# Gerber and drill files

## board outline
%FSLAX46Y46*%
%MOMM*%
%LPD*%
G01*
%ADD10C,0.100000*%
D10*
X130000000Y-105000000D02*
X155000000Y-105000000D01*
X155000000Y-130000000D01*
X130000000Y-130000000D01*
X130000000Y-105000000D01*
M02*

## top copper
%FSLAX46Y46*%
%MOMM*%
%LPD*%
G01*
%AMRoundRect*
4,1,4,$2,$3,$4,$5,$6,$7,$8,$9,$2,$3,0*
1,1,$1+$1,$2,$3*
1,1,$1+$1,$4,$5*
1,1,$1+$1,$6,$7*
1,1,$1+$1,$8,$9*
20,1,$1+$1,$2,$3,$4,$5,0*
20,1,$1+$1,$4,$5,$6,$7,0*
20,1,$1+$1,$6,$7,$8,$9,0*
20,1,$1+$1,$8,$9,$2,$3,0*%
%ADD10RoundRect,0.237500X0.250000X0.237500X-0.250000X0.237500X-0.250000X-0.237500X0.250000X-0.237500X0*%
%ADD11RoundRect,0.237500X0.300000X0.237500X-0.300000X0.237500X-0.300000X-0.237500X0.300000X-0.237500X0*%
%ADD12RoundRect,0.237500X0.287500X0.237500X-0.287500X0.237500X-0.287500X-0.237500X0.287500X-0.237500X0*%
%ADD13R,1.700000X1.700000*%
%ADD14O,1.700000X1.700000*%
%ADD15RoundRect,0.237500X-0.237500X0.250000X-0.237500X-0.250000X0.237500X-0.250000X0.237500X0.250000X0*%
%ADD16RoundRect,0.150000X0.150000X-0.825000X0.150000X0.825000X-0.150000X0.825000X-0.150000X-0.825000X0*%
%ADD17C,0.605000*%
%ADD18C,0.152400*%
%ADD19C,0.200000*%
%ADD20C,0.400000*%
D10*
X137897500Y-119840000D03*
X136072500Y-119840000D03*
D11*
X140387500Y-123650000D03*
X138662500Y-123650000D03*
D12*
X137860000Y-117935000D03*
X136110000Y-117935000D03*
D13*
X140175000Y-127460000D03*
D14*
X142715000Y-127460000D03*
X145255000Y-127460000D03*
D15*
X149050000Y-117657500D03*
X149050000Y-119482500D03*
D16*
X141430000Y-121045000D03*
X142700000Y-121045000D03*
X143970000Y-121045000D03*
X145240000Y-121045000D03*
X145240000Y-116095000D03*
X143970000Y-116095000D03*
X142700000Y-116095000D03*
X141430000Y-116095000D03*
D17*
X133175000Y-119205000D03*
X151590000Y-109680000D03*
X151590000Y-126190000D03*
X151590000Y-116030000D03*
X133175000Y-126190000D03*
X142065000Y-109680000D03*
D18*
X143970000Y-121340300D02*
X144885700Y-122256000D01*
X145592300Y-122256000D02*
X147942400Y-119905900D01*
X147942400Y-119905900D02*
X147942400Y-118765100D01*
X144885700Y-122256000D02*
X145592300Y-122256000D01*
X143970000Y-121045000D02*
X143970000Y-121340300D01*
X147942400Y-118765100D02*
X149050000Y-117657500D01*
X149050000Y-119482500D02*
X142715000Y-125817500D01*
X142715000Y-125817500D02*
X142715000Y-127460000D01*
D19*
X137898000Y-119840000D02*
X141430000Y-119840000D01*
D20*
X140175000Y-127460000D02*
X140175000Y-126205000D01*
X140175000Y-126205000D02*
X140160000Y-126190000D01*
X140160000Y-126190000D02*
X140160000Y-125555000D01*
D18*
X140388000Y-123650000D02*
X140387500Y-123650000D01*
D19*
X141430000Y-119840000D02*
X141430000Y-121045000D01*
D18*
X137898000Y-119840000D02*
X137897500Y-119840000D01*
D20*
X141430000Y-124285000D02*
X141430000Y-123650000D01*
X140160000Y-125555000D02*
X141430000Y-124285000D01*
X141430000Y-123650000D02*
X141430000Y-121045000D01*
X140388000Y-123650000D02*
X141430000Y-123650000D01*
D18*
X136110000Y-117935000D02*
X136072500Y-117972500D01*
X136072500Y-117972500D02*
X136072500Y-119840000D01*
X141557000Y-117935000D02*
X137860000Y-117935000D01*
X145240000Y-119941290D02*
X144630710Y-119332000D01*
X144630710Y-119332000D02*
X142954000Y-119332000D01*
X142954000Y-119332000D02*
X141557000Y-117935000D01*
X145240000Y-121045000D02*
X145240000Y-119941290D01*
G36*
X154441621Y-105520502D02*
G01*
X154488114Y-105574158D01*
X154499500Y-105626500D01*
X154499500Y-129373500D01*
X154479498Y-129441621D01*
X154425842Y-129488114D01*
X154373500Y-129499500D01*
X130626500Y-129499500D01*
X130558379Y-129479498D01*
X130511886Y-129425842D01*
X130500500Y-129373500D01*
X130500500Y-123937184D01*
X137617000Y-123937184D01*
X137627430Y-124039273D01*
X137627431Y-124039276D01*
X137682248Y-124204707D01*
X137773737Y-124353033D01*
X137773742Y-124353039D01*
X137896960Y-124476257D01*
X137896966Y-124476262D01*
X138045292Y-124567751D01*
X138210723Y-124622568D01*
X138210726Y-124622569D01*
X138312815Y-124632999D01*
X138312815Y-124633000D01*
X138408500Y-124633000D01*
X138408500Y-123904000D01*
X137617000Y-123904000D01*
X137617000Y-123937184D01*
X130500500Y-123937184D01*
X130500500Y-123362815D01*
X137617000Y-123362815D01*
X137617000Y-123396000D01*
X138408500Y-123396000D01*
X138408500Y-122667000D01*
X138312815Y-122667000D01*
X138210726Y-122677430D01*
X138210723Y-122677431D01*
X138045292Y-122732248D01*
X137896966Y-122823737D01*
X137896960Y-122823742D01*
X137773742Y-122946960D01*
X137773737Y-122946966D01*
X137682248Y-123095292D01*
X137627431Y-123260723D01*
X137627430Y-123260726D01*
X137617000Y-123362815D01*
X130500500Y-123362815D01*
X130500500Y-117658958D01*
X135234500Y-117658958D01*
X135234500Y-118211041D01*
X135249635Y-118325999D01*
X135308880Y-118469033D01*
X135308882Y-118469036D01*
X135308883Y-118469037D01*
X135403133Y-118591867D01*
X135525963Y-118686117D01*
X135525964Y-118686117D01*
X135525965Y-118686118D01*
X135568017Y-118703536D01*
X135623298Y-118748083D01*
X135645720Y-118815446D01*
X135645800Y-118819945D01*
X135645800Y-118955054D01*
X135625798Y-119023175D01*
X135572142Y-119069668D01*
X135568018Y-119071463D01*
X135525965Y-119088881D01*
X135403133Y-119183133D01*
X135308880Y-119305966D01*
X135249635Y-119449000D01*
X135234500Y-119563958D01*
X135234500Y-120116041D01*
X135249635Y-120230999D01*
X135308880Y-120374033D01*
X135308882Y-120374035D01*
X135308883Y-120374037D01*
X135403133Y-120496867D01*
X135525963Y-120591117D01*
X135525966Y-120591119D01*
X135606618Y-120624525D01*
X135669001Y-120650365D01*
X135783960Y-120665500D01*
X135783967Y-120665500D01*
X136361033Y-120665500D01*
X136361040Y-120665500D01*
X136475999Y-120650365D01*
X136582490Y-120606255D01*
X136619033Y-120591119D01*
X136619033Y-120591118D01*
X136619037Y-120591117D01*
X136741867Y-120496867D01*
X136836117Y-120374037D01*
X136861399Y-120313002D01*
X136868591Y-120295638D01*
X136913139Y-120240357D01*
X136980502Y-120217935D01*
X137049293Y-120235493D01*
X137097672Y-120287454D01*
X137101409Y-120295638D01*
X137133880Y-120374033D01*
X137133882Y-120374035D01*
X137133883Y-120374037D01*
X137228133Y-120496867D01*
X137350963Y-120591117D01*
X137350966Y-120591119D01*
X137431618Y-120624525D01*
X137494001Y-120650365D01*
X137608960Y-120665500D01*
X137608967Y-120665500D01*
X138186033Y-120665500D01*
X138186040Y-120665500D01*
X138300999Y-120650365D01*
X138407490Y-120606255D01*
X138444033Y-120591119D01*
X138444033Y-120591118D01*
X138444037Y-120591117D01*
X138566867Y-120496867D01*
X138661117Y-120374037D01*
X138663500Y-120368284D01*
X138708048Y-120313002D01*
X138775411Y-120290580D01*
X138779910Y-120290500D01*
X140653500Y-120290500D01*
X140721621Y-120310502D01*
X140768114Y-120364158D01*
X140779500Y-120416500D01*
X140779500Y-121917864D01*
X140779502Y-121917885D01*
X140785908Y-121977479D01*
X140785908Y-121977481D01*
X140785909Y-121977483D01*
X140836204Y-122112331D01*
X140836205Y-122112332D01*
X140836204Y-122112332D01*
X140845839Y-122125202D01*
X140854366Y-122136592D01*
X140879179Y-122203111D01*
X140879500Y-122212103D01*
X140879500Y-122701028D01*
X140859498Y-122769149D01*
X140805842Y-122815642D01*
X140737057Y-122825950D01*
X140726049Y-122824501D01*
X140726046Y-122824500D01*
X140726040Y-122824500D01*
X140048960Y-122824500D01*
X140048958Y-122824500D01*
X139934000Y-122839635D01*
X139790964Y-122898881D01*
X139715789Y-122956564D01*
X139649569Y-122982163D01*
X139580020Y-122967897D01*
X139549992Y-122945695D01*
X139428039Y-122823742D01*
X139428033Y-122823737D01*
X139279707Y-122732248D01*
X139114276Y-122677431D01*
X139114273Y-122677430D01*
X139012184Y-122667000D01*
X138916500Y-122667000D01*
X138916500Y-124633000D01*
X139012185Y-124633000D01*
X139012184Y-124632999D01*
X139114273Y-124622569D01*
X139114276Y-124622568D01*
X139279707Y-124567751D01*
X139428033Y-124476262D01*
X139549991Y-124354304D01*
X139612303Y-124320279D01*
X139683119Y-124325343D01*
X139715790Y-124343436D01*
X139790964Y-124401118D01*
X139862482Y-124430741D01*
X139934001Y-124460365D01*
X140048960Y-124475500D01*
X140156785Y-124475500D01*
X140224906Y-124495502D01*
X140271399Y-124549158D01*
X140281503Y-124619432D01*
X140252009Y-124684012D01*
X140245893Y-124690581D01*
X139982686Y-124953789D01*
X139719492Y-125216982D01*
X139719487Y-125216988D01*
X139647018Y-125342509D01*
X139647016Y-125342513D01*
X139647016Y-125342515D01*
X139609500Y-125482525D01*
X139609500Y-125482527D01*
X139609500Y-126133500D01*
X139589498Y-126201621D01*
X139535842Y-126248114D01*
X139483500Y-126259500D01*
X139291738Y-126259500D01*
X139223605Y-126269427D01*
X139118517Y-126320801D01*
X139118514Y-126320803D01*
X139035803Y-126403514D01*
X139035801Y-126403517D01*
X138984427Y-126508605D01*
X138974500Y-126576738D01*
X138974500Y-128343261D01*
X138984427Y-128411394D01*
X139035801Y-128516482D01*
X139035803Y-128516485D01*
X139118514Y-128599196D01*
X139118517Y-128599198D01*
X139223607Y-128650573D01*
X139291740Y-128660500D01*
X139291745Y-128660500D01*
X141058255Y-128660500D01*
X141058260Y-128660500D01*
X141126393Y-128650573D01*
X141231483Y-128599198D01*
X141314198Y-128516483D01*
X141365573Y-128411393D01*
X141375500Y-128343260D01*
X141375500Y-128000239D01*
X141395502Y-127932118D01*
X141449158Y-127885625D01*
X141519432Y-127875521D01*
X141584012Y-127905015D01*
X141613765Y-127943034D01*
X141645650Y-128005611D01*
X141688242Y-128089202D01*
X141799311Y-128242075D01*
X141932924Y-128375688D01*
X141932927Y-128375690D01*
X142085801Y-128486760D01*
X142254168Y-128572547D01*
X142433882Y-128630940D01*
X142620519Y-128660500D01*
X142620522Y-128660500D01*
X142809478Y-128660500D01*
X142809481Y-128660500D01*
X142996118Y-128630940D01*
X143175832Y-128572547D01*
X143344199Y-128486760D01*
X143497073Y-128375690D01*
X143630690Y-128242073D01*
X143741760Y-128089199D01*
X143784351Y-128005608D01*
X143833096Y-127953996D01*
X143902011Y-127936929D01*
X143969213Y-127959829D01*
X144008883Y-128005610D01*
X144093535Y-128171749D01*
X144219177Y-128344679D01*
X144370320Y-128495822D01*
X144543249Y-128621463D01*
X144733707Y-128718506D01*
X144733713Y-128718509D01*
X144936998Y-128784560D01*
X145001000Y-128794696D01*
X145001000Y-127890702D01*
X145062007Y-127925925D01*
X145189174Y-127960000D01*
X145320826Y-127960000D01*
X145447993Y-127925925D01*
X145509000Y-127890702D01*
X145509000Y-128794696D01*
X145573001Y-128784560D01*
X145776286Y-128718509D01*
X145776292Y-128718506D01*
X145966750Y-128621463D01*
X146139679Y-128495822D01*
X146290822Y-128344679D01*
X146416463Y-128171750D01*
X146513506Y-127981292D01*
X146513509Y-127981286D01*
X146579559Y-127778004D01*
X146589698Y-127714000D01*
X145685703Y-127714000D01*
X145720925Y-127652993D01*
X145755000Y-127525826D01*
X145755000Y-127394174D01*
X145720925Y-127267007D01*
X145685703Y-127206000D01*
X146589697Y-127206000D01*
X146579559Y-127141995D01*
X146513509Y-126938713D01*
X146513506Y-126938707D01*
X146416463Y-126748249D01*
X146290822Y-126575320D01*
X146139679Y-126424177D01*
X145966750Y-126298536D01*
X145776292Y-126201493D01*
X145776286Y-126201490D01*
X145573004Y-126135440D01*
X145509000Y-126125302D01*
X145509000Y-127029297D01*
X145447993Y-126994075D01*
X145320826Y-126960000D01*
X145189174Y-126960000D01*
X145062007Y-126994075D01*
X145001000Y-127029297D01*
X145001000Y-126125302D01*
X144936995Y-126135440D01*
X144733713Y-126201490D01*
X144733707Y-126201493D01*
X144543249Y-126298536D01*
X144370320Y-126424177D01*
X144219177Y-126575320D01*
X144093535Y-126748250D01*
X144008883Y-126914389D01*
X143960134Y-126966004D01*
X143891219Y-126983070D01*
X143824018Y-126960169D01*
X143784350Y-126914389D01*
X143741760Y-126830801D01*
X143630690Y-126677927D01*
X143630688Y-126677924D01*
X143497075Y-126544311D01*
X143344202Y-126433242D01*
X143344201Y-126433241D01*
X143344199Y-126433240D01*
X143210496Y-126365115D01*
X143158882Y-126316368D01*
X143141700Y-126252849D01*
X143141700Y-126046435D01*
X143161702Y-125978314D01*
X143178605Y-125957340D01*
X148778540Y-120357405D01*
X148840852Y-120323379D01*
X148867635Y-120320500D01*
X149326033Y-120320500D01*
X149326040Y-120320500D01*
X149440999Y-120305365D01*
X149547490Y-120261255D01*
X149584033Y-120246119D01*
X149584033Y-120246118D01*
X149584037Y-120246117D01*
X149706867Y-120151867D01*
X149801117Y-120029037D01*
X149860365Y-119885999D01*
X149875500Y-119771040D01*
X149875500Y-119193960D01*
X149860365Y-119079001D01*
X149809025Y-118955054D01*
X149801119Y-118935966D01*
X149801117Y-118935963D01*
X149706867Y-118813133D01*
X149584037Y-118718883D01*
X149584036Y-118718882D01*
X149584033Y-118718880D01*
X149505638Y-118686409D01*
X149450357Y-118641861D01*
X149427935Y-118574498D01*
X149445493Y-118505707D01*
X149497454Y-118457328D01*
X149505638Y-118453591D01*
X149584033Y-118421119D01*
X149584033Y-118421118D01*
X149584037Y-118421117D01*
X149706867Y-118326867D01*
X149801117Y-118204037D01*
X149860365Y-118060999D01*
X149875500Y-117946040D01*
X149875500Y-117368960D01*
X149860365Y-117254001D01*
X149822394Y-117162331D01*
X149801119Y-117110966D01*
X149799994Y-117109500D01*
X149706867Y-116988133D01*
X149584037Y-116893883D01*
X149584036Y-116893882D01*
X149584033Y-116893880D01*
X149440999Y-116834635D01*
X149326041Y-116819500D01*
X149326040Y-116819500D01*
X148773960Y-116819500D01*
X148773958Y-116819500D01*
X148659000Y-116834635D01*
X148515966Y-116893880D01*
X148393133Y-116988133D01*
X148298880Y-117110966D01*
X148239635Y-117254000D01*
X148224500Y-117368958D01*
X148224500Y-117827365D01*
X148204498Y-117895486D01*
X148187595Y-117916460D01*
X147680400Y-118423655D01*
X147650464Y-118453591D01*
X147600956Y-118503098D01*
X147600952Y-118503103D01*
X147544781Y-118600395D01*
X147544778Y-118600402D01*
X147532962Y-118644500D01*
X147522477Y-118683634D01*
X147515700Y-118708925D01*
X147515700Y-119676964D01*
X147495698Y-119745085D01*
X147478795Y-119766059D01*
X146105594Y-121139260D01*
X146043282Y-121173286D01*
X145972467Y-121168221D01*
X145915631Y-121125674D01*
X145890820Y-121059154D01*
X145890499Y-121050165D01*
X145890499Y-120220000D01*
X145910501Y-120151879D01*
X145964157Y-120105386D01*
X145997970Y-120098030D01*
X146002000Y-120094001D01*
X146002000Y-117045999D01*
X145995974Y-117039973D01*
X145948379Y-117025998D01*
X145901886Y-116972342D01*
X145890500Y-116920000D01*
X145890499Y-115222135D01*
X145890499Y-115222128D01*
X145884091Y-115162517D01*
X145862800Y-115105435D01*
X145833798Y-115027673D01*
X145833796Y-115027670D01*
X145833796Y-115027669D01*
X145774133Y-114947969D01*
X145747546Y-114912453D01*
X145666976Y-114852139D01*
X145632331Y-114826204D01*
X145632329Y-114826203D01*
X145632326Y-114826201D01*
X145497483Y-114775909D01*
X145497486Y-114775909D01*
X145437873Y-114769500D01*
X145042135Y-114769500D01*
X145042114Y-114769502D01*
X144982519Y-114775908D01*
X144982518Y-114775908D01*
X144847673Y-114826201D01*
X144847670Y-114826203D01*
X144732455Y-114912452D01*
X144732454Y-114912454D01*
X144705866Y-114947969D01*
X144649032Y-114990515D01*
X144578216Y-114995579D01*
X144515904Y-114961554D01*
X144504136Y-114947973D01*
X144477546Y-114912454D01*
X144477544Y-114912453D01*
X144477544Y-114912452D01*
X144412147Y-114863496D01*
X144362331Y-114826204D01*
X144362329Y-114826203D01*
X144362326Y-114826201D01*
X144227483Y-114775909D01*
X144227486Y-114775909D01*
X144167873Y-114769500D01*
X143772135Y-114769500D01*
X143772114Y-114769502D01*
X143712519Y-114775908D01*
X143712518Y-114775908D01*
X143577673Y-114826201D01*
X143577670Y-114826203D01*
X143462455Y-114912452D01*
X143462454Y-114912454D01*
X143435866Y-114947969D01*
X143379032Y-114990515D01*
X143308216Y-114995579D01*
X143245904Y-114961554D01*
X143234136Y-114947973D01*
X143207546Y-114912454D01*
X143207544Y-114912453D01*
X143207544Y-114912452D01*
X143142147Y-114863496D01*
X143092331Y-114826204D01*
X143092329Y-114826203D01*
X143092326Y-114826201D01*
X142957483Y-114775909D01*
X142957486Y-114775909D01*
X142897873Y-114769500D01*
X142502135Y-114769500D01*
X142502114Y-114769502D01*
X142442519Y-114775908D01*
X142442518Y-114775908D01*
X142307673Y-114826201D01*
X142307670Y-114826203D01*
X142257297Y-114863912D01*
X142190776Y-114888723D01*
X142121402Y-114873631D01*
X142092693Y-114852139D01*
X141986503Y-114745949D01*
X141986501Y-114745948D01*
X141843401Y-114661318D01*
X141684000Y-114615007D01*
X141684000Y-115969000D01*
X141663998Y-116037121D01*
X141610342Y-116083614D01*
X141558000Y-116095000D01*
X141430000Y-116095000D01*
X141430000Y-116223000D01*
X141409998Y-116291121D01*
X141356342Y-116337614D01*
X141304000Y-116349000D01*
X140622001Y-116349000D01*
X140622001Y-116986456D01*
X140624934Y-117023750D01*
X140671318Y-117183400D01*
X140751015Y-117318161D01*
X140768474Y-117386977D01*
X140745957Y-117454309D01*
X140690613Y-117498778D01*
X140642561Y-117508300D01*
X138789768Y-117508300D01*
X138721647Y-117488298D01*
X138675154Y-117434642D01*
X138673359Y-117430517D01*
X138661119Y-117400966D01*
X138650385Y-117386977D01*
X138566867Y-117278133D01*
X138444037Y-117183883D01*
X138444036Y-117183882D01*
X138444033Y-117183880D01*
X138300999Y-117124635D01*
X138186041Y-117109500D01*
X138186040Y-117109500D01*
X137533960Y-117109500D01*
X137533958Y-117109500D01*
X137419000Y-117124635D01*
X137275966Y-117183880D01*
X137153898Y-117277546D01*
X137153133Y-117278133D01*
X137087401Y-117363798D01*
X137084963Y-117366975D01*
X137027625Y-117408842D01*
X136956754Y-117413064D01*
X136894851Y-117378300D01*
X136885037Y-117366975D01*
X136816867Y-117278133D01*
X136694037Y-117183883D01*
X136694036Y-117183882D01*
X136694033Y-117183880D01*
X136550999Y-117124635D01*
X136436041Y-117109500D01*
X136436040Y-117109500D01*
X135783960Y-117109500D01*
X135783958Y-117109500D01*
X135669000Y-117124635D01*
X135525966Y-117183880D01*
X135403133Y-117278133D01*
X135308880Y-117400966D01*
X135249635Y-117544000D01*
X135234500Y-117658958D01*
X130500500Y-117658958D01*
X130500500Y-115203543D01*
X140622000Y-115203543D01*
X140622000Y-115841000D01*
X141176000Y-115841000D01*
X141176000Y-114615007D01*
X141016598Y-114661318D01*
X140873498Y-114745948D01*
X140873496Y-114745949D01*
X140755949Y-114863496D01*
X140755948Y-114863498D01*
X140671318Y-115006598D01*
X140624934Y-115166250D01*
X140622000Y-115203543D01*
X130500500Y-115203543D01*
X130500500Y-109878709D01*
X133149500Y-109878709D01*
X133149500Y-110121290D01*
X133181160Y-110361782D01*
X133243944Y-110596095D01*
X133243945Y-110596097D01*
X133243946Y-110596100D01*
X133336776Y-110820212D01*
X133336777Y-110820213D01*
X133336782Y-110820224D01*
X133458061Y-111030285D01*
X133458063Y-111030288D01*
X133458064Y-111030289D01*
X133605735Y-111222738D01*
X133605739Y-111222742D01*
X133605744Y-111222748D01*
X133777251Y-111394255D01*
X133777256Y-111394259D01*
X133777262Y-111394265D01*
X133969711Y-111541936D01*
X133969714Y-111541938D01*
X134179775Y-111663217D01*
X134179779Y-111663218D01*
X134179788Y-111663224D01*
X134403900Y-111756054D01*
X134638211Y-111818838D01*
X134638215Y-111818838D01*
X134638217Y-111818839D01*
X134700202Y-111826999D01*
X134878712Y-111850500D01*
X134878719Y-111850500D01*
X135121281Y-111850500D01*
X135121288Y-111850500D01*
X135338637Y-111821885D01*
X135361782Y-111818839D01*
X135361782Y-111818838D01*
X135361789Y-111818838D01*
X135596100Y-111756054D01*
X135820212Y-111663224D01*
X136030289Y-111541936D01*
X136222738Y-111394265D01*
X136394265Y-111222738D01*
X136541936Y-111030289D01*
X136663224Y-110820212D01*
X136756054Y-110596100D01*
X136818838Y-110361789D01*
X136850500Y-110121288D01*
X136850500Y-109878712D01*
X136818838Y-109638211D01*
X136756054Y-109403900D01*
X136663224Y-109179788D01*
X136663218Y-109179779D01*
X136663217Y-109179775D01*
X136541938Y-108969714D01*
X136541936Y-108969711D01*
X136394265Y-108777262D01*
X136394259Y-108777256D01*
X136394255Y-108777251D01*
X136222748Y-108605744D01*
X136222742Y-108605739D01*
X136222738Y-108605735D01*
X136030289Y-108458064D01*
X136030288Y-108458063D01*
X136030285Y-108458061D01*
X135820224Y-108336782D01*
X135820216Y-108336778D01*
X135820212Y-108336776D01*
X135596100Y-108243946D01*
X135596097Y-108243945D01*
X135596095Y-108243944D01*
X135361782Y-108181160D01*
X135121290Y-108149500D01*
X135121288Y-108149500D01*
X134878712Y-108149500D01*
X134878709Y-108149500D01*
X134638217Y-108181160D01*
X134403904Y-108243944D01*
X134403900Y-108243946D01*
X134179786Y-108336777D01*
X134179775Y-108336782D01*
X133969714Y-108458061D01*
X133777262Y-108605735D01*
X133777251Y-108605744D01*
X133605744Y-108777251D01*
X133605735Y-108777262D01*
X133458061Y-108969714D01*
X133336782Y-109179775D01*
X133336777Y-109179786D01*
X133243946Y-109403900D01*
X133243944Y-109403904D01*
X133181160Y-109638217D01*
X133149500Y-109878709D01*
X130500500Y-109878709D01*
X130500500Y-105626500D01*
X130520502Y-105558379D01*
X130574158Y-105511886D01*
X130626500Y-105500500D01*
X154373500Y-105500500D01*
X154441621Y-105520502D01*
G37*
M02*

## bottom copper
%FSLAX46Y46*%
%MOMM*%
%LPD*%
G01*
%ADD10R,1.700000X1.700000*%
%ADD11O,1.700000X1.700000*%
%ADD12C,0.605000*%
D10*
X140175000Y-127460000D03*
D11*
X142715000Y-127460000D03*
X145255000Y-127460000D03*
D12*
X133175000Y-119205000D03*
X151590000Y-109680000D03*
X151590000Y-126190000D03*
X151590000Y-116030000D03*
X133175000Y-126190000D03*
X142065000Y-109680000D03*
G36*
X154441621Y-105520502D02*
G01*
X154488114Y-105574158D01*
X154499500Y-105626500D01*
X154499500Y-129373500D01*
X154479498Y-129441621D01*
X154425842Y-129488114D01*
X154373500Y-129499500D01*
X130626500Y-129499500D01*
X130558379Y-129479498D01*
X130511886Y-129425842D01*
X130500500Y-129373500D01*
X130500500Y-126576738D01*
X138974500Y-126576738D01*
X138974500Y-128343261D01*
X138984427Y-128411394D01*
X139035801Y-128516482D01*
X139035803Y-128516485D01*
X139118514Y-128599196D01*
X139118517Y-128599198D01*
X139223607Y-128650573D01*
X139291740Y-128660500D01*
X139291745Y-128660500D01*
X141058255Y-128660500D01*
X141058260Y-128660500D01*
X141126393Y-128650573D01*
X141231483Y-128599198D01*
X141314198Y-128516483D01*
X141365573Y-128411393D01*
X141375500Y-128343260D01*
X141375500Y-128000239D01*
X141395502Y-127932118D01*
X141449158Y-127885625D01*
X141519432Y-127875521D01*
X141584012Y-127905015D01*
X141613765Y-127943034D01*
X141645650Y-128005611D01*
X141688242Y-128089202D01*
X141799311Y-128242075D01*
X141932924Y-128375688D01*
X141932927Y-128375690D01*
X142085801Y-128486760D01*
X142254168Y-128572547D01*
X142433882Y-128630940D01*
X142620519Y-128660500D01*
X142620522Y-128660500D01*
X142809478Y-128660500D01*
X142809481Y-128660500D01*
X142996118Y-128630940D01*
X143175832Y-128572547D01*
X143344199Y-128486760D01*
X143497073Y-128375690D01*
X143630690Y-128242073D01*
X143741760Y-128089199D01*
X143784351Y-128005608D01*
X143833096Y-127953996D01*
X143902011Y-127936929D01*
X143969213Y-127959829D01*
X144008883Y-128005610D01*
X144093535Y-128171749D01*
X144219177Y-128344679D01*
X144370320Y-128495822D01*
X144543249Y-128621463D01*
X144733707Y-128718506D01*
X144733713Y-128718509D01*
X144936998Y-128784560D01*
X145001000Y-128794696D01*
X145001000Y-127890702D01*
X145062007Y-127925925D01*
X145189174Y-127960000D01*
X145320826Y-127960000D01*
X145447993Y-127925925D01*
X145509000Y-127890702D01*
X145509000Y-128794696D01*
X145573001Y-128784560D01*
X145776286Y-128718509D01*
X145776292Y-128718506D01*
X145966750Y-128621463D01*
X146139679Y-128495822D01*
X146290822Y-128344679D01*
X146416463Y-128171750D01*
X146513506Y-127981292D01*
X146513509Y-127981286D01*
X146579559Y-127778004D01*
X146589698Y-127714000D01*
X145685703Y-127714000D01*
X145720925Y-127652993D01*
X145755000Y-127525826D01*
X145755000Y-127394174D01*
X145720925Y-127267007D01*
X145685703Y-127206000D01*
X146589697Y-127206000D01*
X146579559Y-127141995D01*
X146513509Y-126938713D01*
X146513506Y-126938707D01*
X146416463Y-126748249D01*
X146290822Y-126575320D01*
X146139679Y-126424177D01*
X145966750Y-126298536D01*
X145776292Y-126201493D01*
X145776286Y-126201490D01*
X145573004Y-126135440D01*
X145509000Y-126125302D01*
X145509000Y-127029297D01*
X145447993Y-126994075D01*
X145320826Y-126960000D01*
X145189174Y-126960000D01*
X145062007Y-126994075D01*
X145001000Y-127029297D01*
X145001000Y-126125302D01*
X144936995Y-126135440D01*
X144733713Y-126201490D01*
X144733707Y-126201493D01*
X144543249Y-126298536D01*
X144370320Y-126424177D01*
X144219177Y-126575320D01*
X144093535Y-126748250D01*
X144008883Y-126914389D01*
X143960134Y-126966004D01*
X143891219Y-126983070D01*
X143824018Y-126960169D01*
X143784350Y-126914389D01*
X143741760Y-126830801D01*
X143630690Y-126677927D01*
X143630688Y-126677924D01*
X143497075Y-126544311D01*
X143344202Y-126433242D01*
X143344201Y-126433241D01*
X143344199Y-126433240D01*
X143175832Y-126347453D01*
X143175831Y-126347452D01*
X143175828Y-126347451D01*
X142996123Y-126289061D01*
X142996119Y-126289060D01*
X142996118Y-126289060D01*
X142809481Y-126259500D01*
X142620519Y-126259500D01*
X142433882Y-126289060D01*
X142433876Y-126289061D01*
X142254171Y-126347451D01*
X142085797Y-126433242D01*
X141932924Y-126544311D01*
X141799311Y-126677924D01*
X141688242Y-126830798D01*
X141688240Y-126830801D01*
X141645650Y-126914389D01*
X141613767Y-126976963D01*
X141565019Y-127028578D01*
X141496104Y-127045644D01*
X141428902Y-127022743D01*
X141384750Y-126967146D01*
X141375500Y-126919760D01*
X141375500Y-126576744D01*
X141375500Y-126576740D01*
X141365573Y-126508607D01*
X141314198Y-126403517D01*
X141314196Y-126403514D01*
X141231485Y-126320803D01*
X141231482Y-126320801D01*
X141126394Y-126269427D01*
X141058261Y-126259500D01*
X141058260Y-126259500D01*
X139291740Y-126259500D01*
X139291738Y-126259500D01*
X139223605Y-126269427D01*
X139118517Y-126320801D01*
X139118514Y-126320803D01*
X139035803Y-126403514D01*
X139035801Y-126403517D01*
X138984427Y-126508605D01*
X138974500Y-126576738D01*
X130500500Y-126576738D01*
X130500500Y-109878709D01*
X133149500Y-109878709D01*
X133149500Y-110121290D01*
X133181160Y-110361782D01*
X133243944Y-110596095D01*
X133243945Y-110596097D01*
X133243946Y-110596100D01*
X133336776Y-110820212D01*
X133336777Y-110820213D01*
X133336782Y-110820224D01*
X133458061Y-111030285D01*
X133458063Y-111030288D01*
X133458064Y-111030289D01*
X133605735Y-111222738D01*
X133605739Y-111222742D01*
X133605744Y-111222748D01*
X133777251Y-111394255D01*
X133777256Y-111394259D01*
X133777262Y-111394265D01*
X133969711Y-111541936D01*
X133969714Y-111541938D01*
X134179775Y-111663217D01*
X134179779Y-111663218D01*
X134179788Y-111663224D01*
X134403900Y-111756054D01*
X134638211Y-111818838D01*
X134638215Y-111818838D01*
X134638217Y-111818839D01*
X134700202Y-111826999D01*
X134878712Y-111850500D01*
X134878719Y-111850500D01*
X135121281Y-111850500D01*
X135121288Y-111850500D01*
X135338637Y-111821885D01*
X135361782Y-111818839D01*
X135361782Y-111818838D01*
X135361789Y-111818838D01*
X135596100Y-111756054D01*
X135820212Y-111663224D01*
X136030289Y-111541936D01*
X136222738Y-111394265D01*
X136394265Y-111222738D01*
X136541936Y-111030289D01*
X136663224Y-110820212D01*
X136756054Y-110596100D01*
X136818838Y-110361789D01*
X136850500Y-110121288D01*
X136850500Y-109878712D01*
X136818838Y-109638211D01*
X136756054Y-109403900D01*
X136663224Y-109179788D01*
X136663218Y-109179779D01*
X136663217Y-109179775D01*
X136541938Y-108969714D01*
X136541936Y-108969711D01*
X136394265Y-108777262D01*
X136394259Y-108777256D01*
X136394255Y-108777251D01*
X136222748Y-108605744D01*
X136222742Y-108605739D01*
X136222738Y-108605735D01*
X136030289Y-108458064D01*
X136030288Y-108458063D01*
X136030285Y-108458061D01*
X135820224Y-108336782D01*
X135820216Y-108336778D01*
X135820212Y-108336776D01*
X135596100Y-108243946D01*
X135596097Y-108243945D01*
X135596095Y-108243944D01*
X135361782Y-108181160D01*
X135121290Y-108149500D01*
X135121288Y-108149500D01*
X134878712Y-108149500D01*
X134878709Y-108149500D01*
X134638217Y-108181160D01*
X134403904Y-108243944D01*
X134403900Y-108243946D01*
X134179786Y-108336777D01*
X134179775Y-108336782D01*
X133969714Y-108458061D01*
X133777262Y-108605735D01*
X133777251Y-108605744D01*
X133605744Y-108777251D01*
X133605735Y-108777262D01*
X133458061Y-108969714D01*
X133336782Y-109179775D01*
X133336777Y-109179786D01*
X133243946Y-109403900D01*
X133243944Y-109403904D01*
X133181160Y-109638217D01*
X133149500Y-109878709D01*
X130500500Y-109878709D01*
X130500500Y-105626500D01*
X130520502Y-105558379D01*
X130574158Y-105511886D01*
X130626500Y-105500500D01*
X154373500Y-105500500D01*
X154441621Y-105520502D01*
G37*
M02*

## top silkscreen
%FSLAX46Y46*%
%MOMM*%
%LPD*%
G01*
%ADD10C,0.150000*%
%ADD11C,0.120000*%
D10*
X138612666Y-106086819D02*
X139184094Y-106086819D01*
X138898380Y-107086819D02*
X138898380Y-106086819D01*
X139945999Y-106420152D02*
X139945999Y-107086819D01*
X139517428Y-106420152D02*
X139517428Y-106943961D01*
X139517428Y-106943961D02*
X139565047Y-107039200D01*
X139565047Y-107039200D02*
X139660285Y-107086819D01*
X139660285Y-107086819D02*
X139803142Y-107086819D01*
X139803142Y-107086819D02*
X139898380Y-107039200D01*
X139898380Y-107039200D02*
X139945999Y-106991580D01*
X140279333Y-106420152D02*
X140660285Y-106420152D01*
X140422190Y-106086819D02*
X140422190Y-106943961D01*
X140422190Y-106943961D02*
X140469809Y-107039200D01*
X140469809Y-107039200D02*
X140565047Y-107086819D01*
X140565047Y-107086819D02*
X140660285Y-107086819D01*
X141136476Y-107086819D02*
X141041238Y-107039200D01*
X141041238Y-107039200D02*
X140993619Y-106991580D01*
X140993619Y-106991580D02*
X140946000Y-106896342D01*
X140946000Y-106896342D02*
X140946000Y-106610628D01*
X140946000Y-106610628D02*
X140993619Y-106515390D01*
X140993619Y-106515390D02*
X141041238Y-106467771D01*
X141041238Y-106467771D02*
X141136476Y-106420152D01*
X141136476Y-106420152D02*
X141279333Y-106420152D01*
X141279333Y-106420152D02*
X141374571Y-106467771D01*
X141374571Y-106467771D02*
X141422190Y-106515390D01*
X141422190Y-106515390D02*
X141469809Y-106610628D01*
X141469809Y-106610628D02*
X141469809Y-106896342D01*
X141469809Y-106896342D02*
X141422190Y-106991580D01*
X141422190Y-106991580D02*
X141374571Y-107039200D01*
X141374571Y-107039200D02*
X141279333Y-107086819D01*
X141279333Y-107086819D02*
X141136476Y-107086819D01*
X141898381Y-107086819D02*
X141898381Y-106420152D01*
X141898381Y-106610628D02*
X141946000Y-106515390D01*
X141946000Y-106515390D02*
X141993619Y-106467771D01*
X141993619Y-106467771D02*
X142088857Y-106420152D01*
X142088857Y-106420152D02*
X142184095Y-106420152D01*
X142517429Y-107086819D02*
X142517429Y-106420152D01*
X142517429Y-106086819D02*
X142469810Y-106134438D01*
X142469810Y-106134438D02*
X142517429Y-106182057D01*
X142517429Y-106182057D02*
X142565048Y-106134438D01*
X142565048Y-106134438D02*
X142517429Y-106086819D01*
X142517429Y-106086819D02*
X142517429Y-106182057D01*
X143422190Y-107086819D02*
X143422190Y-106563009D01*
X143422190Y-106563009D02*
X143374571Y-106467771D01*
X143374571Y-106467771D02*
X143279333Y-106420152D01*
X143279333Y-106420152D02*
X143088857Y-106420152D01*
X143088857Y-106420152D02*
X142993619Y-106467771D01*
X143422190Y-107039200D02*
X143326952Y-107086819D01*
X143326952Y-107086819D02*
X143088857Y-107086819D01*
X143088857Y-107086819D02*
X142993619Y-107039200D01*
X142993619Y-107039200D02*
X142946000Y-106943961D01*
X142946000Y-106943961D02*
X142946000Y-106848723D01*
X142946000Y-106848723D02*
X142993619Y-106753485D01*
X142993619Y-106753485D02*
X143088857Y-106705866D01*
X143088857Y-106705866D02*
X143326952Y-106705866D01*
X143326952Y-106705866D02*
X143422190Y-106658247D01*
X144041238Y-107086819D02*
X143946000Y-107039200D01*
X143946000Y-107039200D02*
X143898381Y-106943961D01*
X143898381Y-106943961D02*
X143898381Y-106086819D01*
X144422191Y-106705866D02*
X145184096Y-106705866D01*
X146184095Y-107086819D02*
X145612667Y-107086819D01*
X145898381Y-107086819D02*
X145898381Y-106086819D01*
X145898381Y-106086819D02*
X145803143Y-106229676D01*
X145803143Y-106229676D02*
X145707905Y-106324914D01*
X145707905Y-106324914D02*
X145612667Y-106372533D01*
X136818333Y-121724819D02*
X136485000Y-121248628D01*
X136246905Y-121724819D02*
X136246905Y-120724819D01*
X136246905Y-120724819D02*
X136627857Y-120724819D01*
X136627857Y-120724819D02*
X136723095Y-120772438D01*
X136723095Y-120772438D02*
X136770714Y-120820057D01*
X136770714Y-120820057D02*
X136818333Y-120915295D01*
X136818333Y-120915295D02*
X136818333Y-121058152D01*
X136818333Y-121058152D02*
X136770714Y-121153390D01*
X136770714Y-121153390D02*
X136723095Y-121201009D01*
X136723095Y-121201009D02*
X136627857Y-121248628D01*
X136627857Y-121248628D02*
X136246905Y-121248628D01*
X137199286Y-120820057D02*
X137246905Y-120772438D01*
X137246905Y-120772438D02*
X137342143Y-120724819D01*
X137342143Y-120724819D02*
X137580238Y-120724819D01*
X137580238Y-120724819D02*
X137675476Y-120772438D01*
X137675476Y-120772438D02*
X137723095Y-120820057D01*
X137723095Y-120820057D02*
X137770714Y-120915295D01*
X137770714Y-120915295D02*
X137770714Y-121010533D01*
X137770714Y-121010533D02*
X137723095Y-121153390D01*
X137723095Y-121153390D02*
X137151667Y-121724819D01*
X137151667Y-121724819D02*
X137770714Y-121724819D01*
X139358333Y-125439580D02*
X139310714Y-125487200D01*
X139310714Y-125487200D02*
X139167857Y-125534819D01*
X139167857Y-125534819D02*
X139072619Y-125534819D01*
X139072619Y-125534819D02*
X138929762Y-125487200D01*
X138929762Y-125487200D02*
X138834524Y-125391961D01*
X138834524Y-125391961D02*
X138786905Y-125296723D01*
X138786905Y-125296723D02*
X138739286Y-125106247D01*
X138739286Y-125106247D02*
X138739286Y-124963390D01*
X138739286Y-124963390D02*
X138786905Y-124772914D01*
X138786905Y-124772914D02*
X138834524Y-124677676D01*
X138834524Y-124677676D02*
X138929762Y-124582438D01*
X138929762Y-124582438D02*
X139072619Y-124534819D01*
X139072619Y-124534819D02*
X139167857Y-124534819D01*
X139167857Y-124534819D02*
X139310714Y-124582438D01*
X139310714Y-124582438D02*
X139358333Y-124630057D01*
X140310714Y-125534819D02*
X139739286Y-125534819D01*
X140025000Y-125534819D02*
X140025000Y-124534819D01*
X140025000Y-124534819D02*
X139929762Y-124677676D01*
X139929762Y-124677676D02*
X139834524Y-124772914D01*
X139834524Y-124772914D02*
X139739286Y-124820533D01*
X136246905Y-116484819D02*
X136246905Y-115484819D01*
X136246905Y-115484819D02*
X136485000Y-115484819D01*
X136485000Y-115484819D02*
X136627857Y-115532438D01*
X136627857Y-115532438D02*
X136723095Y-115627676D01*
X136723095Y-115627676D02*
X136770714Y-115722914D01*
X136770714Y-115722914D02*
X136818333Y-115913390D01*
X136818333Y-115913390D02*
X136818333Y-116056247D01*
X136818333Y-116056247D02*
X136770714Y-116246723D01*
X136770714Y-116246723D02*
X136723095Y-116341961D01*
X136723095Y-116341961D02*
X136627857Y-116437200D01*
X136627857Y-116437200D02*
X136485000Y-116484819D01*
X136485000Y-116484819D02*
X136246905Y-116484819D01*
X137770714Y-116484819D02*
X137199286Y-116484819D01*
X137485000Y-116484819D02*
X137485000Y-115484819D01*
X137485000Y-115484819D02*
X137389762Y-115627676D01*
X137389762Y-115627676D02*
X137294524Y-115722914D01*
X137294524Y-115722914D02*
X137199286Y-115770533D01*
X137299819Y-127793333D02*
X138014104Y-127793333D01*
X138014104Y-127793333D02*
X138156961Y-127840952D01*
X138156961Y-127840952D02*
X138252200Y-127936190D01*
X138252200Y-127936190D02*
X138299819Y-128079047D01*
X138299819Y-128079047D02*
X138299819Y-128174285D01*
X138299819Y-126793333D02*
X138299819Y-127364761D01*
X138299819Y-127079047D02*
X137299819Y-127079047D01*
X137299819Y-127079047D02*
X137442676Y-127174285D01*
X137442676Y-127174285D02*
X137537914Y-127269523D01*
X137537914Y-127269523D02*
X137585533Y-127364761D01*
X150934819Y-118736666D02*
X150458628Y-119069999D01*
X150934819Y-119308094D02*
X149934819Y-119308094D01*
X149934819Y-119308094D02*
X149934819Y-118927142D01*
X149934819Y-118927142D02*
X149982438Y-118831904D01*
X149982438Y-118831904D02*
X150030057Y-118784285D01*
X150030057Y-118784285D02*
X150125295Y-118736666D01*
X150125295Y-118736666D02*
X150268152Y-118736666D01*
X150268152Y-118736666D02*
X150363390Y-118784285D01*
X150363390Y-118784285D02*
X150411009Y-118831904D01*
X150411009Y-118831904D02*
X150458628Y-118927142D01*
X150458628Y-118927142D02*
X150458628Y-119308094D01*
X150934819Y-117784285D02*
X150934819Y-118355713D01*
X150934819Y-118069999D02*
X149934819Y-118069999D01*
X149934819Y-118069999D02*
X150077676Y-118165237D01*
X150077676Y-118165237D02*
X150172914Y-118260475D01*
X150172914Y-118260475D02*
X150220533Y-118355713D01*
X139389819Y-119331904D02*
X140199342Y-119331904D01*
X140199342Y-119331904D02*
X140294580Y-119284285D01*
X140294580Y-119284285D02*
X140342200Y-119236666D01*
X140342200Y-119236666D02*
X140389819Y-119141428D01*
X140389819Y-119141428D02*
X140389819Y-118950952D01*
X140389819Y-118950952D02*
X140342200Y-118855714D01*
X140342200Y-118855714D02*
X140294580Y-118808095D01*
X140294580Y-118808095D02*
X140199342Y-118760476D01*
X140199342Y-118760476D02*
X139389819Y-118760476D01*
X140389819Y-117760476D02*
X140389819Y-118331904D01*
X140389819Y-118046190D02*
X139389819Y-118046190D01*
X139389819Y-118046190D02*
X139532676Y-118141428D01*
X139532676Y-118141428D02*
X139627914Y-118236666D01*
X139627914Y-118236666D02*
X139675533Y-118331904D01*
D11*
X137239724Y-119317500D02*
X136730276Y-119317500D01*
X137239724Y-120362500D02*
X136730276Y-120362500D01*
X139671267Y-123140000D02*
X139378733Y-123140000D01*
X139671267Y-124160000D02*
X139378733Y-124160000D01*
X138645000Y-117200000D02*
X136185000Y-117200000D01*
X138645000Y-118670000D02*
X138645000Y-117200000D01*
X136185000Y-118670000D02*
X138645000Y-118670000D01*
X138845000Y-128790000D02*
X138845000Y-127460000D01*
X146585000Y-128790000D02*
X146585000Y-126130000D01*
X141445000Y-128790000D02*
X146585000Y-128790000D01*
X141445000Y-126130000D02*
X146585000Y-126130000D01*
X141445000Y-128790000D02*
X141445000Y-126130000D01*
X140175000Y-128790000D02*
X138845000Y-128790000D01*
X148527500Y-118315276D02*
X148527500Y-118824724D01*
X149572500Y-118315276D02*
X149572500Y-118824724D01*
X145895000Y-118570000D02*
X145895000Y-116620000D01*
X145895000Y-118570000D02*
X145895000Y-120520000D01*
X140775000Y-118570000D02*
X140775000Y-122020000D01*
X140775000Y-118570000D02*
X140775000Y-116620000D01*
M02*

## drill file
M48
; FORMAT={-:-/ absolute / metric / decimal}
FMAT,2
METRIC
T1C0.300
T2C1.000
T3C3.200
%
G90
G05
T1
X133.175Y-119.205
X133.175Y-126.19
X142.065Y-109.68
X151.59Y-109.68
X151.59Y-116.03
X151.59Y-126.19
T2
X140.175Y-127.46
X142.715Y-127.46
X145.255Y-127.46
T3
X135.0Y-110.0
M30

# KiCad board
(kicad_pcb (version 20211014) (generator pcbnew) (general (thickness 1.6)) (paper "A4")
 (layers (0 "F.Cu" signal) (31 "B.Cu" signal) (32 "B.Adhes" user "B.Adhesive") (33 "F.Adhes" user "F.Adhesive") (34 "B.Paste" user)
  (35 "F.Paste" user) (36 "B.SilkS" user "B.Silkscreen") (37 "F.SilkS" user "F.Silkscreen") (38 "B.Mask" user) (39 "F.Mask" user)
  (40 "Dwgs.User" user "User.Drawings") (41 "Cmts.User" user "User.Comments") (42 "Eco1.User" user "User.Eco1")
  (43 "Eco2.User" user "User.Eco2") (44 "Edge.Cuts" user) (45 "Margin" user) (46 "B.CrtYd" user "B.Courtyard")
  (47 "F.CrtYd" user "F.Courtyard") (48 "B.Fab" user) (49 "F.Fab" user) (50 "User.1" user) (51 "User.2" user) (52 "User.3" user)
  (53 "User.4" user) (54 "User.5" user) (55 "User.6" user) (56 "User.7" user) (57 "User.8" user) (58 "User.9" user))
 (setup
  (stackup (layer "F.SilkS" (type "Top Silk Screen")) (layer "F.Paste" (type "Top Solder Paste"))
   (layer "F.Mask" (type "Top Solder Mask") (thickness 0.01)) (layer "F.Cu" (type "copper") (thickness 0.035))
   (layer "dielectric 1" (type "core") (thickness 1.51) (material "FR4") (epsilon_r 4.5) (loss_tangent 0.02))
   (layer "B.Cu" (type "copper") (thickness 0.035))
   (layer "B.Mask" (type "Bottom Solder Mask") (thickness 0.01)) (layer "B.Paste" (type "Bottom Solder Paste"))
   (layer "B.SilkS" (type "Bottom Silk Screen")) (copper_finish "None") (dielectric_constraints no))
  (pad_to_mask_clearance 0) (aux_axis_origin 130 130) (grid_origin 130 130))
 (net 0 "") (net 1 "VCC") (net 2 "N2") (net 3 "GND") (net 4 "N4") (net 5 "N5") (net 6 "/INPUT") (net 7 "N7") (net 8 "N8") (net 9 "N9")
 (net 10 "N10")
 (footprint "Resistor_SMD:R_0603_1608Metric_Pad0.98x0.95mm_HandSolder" (layer "F.Cu") (at 136.985 119.84 180)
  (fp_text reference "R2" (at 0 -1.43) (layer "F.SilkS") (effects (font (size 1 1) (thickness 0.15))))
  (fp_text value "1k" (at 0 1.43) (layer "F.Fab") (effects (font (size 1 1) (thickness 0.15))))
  (fp_line (start -0.254724 0.5225) (end 0.254724 0.5225) (layer "F.SilkS") (width 0.12))
  (fp_line (start -0.254724 -0.5225) (end 0.254724 -0.5225) (layer "F.SilkS") (width 0.12))
  (pad "1" smd roundrect (at -0.9125 0 180) (size 0.975 0.95) (layers "F.Cu" "F.Paste" "F.Mask") (roundrect_rratio 0.25) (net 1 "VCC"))
  (pad "2" smd roundrect (at 0.9125 0 180) (size 0.975 0.95) (layers "F.Cu" "F.Paste" "F.Mask") (roundrect_rratio 0.25) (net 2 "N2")))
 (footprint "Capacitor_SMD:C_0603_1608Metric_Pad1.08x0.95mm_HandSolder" (layer "F.Cu") (at 139.525 123.65 180)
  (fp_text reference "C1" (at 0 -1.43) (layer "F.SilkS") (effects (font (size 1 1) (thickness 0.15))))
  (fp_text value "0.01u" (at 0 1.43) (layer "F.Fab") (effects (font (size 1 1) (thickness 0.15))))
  (fp_line (start -0.146267 0.51) (end 0.146267 0.51) (layer "F.SilkS") (width 0.12))
  (fp_line (start -0.146267 -0.51) (end 0.146267 -0.51) (layer "F.SilkS") (width 0.12))
  (pad "1" smd roundrect (at -0.8625 0 180) (size 1.075 0.95) (layers "F.Cu" "F.Paste" "F.Mask") (roundrect_rratio 0.25) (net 1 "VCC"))
  (pad "2" smd roundrect (at 0.8625 0 180) (size 1.075 0.95) (layers "F.Cu" "F.Paste" "F.Mask") (roundrect_rratio 0.25) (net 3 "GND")))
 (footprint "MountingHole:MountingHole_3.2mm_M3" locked (layer "F.Cu") (at 135 110)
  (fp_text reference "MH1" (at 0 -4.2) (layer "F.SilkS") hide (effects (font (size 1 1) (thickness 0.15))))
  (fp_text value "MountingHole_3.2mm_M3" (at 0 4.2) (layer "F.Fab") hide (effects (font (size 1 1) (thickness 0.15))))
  (pad "" np_thru_hole circle locked (at 0 0) (size 3.2 3.2) (drill 3.2) (layers *.Cu *.Mask)))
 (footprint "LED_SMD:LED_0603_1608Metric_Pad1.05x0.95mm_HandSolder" (layer "F.Cu") (at 136.985 117.935 180)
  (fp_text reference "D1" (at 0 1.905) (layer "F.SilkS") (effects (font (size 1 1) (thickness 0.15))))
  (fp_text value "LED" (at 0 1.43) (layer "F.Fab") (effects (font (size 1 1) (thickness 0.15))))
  (fp_line (start -1.66 0.735) (end 0.8 0.735) (layer "F.SilkS") (width 0.12))
  (fp_line (start -1.66 -0.735) (end -1.66 0.735) (layer "F.SilkS") (width 0.12))
  (fp_line (start 0.8 -0.735) (end -1.66 -0.735) (layer "F.SilkS") (width 0.12))
  (pad "1" smd roundrect (at -0.875 0 180) (size 1.05 0.95) (layers "F.Cu" "F.Paste" "F.Mask") (roundrect_rratio 0.25) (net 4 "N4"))
  (pad "2" smd roundrect (at 0.875 0 180) (size 1.05 0.95) (layers "F.Cu" "F.Paste" "F.Mask") (roundrect_rratio 0.25) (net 2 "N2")))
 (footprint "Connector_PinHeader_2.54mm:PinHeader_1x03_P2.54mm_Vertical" (layer "F.Cu") (at 140.175 127.46 90)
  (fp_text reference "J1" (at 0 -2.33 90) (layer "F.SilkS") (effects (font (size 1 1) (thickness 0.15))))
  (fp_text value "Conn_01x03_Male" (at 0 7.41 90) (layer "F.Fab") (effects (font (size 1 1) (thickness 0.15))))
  (fp_line (start -1.33 -1.33) (end 0 -1.33) (layer "F.SilkS") (width 0.12))
  (fp_line (start -1.33 6.41) (end 1.33 6.41) (layer "F.SilkS") (width 0.12))
  (fp_line (start -1.33 1.27) (end -1.33 6.41) (layer "F.SilkS") (width 0.12))
  (fp_line (start 1.33 1.27) (end 1.33 6.41) (layer "F.SilkS") (width 0.12))
  (fp_line (start -1.33 1.27) (end 1.33 1.27) (layer "F.SilkS") (width 0.12))
  (fp_line (start -1.33 0) (end -1.33 -1.33) (layer "F.SilkS") (width 0.12))
  (pad "1" thru_hole rect (at 0 0 90) (size 1.7 1.7) (drill 1) (layers *.Cu *.Mask) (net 1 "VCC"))
  (pad "2" thru_hole oval (at 0 2.54 90) (size 1.7 1.7) (drill 1) (layers *.Cu *.Mask) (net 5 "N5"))
  (pad "3" thru_hole oval (at 0 5.08 90) (size 1.7 1.7) (drill 1) (layers *.Cu *.Mask) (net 3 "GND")))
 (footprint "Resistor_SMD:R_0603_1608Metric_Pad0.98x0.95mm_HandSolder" (layer "F.Cu") (at 149.05 118.57 -90)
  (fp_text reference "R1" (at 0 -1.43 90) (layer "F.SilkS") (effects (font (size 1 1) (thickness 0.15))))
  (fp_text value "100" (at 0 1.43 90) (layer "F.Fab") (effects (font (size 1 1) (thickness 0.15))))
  (fp_line (start -0.254724 0.5225) (end 0.254724 0.5225) (layer "F.SilkS") (width 0.12))
  (fp_line (start -0.254724 -0.5225) (end 0.254724 -0.5225) (layer "F.SilkS") (width 0.12))
  (pad "1" smd roundrect (at -0.9125 0 270) (size 0.975 0.95) (layers "F.Cu" "F.Paste" "F.Mask") (roundrect_rratio 0.25) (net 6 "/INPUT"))
  (pad "2" smd roundrect (at 0.9125 0 270) (size 0.975 0.95) (layers "F.Cu" "F.Paste" "F.Mask") (roundrect_rratio 0.25) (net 5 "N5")))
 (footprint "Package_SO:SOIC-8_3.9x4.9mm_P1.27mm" (layer "F.Cu") (at 143.335 118.57 90)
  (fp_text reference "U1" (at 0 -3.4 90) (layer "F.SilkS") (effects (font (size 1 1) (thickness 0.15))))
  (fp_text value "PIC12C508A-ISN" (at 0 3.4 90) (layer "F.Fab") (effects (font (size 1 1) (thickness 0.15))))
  (fp_line (start 0 2.56) (end 1.95 2.56) (layer "F.SilkS") (width 0.12))
  (fp_line (start 0 2.56) (end -1.95 2.56) (layer "F.SilkS") (width 0.12))
  (fp_line (start 0 -2.56) (end -3.45 -2.56) (layer "F.SilkS") (width 0.12))
  (fp_line (start 0 -2.56) (end 1.95 -2.56) (layer "F.SilkS") (width 0.12))
  (pad "1" smd roundrect (at -2.475 -1.905 90) (size 1.95 0.6) (layers "F.Cu" "F.Paste" "F.Mask") (roundrect_rratio 0.25) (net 1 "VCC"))
  (pad "2" smd roundrect (at -2.475 -0.635 90) (size 1.95 0.6) (layers "F.Cu" "F.Paste" "F.Mask") (roundrect_rratio 0.25) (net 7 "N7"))
  (pad "3" smd roundrect (at -2.475 0.635 90) (size 1.95 0.6) (layers "F.Cu" "F.Paste" "F.Mask") (roundrect_rratio 0.25) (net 6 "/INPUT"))
  (pad "4" smd roundrect (at -2.475 1.905 90) (size 1.95 0.6) (layers "F.Cu" "F.Paste" "F.Mask") (roundrect_rratio 0.25) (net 4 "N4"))
  (pad "5" smd roundrect (at 2.475 1.905 90) (size 1.95 0.6) (layers "F.Cu" "F.Paste" "F.Mask") (roundrect_rratio 0.25) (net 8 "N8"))
  (pad "6" smd roundrect (at 2.475 0.635 90) (size 1.95 0.6) (layers "F.Cu" "F.Paste" "F.Mask") (roundrect_rratio 0.25) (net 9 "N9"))
  (pad "7" smd roundrect (at 2.475 -0.635 90) (size 1.95 0.6) (layers "F.Cu" "F.Paste" "F.Mask") (roundrect_rratio 0.25) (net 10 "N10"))
  (pad "8" smd roundrect (at 2.475 -1.905 90) (size 1.95 0.6) (layers "F.Cu" "F.Paste" "F.Mask") (roundrect_rratio 0.25) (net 3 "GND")))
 (gr_rect locked (start 130 130) (end 155 105) (layer "Edge.Cuts") (width 0.1) (fill none))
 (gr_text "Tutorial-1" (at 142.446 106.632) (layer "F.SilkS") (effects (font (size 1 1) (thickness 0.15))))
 (segment (start 143.97 121.3403) (end 144.8857 122.256) (width 0.1524) (layer "F.Cu") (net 6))
 (segment (start 145.5923 122.256) (end 147.9424 119.9059) (width 0.1524) (layer "F.Cu") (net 6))
 (segment (start 147.9424 119.9059) (end 147.9424 118.7651) (width 0.1524) (layer "F.Cu") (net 6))
 (segment (start 144.8857 122.256) (end 145.5923 122.256) (width 0.1524) (layer "F.Cu") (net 6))
 (segment (start 143.97 121.045) (end 143.97 121.3403) (width 0.1524) (layer "F.Cu") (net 6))
 (segment (start 147.9424 118.7651) (end 149.05 117.6575) (width 0.1524) (layer "F.Cu") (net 6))
 (segment (start 149.05 119.4825) (end 142.715 125.8175) (width 0.1524) (layer "F.Cu") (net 5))
 (segment (start 142.715 125.8175) (end 142.715 127.46) (width 0.1524) (layer "F.Cu") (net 5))
 (segment (start 137.898 119.84) (end 141.43 119.84) (width 0.2) (layer "F.Cu") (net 1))
 (segment (start 140.175 127.46) (end 140.175 126.205) (width 0.4) (layer "F.Cu") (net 1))
 (segment (start 140.175 126.205) (end 140.16 126.19) (width 0.4) (layer "F.Cu") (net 1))
 (segment (start 140.16 126.19) (end 140.16 125.555) (width 0.4) (layer "F.Cu") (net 1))
 (segment (start 140.388 123.65) (end 140.3875 123.65) (width 0.1524) (layer "F.Cu") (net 1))
 (segment (start 141.43 119.84) (end 141.43 121.045) (width 0.2) (layer "F.Cu") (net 1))
 (segment (start 137.898 119.84) (end 137.8975 119.84) (width 0.1524) (layer "F.Cu") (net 1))
 (segment (start 141.43 124.285) (end 141.43 123.65) (width 0.4) (layer "F.Cu") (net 1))
 (segment (start 140.16 125.555) (end 141.43 124.285) (width 0.4) (layer "F.Cu") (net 1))
 (segment (start 141.43 123.65) (end 141.43 121.045) (width 0.4) (layer "F.Cu") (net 1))
 (segment (start 140.388 123.65) (end 141.43 123.65) (width 0.4) (layer "F.Cu") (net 1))
 (segment (start 136.11 117.935) (end 136.0725 117.9725) (width 0.1524) (layer "F.Cu") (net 2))
 (segment (start 136.0725 117.9725) (end 136.0725 119.84) (width 0.1524) (layer "F.Cu") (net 2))
 (segment (start 141.557 117.935) (end 137.86 117.935) (width 0.1524) (layer "F.Cu") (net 4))
 (segment (start 145.24 119.94129) (end 144.63071 119.332) (width 0.1524) (layer "F.Cu") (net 4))
 (segment (start 144.63071 119.332) (end 142.954 119.332) (width 0.1524) (layer "F.Cu") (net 4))
 (segment (start 142.954 119.332) (end 141.557 117.935) (width 0.1524) (layer "F.Cu") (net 4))
 (segment (start 145.24 121.045) (end 145.24 119.94129) (width 0.1524) (layer "F.Cu") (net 4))
 (via (at 133.175 119.205) (size 0.605) (drill 0.3) (layers "F.Cu" "B.Cu") (free) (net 3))
 (via (at 151.59 109.68) (size 0.605) (drill 0.3) (layers "F.Cu" "B.Cu") (free) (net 3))
 (via (at 151.59 126.19) (size 0.605) (drill 0.3) (layers "F.Cu" "B.Cu") (free) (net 3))
 (via (at 151.59 116.03) (size 0.605) (drill 0.3) (layers "F.Cu" "B.Cu") (free) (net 3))
 (via (at 133.175 126.19) (size 0.605) (drill 0.3) (layers "F.Cu" "B.Cu") (free) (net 3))
 (via (at 142.065 109.68) (size 0.605) (drill 0.3) (layers "F.Cu" "B.Cu") (free) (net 3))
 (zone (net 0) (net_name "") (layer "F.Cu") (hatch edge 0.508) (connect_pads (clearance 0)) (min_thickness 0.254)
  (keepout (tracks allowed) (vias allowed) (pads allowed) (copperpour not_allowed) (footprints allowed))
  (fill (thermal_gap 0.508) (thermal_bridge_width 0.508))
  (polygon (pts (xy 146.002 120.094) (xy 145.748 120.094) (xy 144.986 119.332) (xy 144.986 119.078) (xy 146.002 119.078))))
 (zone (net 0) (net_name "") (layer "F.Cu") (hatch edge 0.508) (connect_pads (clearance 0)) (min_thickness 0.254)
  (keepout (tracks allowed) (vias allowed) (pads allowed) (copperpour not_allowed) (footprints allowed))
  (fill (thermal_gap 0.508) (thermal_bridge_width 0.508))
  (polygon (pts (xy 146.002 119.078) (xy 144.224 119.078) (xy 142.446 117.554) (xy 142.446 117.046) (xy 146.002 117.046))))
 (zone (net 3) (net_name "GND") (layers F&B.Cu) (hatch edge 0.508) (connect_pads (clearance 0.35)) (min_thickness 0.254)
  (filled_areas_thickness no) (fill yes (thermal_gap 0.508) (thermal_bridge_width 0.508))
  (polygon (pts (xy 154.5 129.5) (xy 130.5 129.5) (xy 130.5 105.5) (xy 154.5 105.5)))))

